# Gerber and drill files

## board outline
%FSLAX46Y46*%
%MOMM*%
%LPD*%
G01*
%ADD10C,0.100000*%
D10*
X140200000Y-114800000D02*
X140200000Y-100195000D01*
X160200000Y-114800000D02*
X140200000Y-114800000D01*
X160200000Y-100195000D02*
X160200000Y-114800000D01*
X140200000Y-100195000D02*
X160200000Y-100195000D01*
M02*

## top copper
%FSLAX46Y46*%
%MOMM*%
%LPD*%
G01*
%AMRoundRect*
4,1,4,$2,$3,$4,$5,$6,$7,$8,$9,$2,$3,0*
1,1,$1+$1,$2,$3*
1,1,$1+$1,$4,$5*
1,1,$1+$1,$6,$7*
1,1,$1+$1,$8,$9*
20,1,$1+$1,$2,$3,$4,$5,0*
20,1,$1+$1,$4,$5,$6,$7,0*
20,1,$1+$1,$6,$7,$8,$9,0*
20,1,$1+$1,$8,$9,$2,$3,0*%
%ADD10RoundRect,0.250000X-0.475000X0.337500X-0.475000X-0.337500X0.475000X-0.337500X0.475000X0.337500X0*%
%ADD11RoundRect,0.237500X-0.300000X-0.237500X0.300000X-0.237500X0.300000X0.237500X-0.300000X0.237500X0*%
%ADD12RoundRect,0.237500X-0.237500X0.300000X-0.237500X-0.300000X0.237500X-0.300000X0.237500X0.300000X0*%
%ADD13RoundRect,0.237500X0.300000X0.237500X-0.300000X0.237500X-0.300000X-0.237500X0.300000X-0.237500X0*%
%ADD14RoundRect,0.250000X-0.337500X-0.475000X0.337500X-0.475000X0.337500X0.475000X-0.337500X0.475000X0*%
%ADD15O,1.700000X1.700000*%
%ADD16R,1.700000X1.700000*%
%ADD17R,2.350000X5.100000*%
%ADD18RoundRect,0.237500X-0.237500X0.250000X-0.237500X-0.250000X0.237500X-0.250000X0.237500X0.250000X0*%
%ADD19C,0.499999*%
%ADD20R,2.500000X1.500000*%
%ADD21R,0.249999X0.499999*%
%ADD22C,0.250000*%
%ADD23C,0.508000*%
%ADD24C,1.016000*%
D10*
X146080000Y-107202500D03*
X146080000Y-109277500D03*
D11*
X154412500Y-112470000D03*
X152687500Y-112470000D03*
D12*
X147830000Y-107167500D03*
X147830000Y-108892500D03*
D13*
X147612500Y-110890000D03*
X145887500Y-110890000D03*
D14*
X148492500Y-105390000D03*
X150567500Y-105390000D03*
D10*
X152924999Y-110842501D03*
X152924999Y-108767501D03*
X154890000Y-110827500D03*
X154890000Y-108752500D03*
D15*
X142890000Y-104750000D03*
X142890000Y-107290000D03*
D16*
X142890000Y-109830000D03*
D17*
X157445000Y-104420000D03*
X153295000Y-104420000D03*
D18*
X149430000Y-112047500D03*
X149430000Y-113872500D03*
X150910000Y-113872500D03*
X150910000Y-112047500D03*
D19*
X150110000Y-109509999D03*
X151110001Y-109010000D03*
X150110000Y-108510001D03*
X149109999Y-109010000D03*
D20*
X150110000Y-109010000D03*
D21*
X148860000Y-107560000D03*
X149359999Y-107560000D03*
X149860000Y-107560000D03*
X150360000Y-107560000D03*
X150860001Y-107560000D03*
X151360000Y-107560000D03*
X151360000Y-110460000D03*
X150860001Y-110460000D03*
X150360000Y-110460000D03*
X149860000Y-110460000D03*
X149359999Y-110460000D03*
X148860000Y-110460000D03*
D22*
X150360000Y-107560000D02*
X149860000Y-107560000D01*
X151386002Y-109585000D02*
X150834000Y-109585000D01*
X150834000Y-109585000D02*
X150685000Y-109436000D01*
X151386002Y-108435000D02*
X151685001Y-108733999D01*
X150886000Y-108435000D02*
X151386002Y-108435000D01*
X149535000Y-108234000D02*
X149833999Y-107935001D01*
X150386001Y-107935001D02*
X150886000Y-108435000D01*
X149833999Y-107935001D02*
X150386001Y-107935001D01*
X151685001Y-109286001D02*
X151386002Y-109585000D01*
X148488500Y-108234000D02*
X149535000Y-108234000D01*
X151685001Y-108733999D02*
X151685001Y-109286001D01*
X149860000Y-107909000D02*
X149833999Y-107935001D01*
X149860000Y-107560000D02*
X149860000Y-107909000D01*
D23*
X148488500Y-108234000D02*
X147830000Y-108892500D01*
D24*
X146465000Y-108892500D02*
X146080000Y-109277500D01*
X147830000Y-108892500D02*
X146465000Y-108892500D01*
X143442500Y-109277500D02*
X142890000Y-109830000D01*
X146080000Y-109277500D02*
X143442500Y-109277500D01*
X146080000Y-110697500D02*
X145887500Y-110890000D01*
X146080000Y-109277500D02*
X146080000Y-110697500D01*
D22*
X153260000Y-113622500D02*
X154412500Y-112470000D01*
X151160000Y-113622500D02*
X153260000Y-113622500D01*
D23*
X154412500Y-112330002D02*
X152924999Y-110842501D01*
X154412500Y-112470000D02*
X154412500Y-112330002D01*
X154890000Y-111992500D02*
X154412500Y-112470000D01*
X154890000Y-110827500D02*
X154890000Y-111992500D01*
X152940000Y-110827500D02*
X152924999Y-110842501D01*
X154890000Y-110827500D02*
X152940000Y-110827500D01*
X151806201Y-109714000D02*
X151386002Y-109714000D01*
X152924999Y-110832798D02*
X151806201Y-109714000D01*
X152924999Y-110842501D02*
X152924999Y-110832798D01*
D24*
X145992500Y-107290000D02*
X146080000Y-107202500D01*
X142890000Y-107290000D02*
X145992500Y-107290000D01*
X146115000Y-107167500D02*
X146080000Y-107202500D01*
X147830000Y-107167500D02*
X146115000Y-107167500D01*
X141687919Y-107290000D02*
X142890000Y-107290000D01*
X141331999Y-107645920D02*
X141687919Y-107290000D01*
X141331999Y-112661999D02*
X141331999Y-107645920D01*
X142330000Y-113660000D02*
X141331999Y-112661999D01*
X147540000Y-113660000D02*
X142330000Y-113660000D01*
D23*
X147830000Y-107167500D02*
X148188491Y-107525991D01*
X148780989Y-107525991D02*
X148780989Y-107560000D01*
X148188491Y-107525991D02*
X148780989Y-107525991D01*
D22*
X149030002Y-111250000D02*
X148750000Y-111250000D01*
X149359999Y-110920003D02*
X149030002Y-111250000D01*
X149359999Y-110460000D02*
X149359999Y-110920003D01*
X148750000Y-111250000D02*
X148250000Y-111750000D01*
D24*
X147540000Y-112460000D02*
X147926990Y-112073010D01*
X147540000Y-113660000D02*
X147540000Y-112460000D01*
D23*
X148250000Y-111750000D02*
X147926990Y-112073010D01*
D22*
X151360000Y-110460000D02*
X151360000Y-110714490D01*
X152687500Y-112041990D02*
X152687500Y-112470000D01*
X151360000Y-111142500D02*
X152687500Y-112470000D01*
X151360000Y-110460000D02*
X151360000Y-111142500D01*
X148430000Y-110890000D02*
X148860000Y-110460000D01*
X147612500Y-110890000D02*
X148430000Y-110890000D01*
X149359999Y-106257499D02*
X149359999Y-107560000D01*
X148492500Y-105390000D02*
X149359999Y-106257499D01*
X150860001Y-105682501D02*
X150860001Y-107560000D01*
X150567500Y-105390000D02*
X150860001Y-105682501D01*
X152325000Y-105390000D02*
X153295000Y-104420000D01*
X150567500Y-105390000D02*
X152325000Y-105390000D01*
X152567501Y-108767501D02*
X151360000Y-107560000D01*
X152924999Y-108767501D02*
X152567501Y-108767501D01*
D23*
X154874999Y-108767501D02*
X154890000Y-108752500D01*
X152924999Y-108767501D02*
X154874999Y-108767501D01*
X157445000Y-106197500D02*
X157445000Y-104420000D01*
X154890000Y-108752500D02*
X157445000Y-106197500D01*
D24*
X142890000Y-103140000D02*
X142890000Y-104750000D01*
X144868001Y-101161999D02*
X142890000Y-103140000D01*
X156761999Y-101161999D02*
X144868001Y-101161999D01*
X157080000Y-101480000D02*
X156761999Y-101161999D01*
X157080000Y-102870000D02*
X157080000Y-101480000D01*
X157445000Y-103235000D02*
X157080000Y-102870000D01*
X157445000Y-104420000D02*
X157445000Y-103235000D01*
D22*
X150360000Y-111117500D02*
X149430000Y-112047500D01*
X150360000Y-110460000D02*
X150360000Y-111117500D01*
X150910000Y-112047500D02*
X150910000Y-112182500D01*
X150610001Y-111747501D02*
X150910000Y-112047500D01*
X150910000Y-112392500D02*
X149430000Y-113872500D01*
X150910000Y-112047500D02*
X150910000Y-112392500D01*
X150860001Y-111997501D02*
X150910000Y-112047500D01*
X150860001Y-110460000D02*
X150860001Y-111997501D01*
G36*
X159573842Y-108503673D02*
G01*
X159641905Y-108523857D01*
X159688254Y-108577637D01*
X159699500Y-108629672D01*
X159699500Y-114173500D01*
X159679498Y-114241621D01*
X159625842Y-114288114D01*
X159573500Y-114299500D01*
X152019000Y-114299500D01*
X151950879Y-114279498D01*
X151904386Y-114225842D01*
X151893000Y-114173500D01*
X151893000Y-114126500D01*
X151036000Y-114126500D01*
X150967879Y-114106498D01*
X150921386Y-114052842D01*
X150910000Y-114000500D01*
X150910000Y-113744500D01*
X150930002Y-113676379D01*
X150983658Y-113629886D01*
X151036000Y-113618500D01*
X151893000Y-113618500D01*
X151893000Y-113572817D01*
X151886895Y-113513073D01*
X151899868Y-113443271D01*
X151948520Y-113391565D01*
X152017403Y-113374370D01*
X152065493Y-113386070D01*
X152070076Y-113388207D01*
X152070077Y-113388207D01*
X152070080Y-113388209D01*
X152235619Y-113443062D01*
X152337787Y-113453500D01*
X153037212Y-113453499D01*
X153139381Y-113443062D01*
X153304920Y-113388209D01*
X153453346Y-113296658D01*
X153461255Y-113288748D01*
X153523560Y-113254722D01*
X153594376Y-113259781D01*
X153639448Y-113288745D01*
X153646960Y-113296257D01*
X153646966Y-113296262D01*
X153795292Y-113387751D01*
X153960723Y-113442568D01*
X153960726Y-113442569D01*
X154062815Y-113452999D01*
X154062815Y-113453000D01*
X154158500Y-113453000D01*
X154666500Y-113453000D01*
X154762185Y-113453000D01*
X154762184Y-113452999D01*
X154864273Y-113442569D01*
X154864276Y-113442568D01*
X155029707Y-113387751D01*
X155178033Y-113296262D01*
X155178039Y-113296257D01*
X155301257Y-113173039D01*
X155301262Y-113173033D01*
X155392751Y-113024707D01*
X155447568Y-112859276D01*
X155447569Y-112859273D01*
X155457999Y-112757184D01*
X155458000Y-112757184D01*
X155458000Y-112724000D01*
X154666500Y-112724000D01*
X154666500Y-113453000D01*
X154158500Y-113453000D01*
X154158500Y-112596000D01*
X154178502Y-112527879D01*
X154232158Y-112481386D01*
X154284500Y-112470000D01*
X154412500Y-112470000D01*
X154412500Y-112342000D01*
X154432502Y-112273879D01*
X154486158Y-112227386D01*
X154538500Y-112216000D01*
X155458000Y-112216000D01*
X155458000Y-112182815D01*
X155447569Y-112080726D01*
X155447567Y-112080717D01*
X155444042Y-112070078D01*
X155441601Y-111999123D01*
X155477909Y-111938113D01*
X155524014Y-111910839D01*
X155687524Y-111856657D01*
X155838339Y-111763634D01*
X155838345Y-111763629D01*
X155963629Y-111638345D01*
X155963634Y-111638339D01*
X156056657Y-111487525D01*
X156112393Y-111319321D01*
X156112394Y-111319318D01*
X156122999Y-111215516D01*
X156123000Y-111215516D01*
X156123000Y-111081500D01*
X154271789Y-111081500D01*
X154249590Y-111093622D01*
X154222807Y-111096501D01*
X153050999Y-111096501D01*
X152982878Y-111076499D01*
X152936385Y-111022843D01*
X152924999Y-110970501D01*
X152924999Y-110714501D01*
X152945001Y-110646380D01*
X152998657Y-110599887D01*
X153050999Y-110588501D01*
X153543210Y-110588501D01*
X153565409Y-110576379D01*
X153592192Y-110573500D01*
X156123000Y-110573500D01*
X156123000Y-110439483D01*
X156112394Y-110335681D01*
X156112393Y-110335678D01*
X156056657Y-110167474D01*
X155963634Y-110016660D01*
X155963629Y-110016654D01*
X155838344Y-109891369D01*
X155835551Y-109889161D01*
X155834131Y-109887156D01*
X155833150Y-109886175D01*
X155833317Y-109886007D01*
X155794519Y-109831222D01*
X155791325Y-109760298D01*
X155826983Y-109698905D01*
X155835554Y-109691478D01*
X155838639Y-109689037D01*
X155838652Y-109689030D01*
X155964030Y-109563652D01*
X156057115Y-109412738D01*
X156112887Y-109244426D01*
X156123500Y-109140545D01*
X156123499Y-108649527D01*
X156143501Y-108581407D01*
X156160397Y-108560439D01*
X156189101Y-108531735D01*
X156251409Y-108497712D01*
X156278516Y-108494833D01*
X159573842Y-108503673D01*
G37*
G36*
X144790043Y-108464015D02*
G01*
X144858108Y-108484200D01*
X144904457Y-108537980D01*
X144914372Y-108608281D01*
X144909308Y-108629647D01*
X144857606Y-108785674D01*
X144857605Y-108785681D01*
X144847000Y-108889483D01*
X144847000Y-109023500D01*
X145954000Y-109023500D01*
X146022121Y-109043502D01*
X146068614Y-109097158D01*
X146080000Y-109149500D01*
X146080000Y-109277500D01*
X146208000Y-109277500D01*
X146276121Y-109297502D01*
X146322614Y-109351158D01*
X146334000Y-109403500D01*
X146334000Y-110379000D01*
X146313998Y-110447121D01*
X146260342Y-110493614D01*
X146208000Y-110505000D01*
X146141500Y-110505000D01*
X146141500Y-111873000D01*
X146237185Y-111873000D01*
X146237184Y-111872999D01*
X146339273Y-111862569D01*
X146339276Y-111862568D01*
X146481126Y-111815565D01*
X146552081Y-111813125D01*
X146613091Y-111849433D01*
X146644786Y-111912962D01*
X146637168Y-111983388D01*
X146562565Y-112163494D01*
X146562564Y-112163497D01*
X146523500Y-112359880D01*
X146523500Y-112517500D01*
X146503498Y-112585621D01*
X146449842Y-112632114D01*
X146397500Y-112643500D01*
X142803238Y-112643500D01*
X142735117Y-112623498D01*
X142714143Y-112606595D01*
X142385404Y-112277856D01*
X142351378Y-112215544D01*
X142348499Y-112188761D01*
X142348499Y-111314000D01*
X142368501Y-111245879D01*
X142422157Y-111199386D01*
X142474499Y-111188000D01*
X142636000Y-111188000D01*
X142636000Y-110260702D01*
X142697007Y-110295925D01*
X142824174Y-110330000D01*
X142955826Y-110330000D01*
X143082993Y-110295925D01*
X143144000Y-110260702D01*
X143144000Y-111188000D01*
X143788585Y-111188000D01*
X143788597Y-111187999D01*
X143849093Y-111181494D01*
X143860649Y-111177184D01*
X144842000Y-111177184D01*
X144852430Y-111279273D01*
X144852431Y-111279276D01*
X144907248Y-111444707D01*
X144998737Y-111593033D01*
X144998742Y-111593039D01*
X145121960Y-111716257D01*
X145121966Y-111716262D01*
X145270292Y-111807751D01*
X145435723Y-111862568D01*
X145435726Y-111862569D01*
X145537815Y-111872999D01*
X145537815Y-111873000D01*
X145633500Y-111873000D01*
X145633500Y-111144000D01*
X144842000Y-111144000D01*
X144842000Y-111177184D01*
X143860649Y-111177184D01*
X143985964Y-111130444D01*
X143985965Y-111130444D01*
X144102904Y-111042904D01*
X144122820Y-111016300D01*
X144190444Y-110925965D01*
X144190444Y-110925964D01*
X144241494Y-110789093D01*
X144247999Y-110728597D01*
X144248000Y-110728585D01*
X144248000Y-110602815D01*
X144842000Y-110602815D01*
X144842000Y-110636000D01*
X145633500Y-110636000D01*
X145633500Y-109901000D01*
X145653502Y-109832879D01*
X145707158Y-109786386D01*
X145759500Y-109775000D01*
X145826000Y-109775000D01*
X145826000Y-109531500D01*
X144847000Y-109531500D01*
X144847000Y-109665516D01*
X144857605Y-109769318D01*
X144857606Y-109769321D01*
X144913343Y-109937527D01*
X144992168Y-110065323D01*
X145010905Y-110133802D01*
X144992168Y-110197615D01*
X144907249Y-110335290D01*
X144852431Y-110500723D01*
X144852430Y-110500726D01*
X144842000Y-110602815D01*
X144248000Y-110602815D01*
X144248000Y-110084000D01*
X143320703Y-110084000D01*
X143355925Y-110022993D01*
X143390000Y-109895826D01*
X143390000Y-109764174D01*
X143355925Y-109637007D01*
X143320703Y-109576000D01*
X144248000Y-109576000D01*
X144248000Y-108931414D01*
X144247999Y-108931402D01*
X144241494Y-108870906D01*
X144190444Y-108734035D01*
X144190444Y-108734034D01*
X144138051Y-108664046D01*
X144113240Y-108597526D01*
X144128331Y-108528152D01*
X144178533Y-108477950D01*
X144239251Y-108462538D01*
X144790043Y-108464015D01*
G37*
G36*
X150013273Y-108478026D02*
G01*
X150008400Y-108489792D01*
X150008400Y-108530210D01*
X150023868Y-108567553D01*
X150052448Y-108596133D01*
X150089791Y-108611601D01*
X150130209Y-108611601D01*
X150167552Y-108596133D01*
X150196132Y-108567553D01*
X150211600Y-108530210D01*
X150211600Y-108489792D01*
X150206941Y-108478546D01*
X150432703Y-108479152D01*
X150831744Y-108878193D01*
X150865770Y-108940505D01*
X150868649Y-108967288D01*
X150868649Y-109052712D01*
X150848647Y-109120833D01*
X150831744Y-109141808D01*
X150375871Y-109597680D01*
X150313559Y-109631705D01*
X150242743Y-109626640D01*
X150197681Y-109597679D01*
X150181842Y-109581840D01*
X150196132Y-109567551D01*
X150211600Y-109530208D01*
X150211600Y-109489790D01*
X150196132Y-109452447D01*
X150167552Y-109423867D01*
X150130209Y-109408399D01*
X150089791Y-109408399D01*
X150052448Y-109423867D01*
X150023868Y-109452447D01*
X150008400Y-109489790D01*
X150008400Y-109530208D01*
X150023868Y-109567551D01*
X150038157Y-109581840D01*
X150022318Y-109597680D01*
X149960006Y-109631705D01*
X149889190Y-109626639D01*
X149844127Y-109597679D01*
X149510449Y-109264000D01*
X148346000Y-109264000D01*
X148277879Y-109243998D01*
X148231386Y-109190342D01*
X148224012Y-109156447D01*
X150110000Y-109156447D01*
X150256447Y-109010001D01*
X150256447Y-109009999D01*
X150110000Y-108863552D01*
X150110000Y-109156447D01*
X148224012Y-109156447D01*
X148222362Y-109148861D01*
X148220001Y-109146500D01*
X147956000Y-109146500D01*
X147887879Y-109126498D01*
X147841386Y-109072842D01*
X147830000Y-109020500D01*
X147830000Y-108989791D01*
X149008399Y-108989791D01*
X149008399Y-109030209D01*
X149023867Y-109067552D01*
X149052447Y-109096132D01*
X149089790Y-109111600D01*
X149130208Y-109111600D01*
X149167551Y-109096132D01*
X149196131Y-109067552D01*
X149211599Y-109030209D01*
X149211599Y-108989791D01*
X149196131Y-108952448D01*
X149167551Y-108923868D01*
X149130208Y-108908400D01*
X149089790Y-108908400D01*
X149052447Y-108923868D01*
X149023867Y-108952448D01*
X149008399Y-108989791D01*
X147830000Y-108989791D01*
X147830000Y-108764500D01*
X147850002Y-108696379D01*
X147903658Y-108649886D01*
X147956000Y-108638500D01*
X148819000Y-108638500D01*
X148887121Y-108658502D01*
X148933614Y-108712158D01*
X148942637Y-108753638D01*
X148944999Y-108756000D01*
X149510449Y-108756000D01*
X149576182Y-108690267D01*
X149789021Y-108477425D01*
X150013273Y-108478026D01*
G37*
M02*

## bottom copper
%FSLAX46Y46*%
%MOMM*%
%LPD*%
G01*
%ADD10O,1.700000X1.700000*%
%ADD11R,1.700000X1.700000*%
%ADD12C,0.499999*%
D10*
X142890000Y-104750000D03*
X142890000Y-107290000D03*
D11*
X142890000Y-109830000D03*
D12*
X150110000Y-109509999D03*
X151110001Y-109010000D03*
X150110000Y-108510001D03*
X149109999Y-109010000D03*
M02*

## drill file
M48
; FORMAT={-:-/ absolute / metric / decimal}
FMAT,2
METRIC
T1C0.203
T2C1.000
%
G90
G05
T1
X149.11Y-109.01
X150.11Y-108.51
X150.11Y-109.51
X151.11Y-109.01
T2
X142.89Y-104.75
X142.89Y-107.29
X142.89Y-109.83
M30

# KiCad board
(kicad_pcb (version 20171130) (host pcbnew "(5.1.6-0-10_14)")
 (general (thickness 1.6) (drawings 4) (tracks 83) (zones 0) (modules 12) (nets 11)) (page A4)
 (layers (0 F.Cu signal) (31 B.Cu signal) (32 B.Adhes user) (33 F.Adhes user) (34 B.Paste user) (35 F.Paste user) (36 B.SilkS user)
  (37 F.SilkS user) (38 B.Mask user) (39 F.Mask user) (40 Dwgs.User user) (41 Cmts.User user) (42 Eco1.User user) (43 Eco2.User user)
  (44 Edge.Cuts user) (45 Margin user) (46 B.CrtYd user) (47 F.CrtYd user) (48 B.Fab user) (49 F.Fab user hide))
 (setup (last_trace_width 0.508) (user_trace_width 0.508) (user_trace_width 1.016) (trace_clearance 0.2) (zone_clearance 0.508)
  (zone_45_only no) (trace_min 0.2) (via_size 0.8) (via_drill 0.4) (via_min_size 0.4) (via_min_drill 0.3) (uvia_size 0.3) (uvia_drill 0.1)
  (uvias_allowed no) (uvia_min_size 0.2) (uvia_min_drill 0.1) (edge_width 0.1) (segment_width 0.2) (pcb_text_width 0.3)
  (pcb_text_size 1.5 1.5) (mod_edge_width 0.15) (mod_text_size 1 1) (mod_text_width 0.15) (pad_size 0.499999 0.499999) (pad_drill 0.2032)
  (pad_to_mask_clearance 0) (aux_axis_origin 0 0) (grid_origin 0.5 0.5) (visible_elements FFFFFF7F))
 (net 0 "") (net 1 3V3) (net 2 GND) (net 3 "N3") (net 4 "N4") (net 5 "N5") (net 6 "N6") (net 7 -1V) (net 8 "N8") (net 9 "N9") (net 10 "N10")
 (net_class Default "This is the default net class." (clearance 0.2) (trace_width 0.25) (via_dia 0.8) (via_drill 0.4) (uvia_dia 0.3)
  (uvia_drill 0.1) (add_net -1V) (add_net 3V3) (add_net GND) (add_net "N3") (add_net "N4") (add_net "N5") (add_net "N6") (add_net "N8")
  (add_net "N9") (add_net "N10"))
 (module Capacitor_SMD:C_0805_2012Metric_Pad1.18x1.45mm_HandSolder (layer F.Cu) (at 146.08 108.24 270)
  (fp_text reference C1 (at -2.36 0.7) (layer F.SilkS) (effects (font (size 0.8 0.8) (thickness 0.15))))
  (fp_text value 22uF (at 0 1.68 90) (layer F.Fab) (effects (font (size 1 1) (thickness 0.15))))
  (pad 1 smd roundrect (at -1.0375 0 270) (size 1.175 1.45) (layers F.Cu F.Paste F.Mask) (roundrect_rratio 0.212766) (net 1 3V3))
  (pad 2 smd roundrect (at 1.0375 0 270) (size 1.175 1.45) (layers F.Cu F.Paste F.Mask) (roundrect_rratio 0.212766) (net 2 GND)))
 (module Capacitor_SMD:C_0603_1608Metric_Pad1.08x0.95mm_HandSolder (layer F.Cu) (at 153.55 112.47)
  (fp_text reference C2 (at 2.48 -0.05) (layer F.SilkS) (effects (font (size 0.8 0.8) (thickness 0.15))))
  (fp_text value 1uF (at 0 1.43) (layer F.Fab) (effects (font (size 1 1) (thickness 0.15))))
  (pad 2 smd roundrect (at 0.8625 0) (size 1.075 0.95) (layers F.Cu F.Paste F.Mask) (roundrect_rratio 0.25) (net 2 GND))
  (pad 1 smd roundrect (at -0.8625 0) (size 1.075 0.95) (layers F.Cu F.Paste F.Mask) (roundrect_rratio 0.25) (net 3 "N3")))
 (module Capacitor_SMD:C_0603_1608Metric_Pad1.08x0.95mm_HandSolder (layer F.Cu) (at 147.83 108.03 270)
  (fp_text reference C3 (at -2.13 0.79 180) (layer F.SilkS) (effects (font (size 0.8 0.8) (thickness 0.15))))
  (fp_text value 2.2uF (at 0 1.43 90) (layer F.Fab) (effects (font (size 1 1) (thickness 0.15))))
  (pad 1 smd roundrect (at -0.8625 0 270) (size 1.075 0.95) (layers F.Cu F.Paste F.Mask) (roundrect_rratio 0.25) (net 1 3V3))
  (pad 2 smd roundrect (at 0.8625 0 270) (size 1.075 0.95) (layers F.Cu F.Paste F.Mask) (roundrect_rratio 0.25) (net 2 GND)))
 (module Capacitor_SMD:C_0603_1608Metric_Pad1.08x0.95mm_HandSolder (layer F.Cu) (at 146.75 110.89 180)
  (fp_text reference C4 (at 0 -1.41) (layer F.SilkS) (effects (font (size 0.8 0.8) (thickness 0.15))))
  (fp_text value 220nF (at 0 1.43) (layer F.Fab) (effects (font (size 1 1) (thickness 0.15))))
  (pad 1 smd roundrect (at -0.8625 0 180) (size 1.075 0.95) (layers F.Cu F.Paste F.Mask) (roundrect_rratio 0.25) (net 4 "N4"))
  (pad 2 smd roundrect (at 0.8625 0 180) (size 1.075 0.95) (layers F.Cu F.Paste F.Mask) (roundrect_rratio 0.25) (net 2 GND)))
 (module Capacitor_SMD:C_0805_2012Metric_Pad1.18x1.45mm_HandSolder (layer F.Cu) (at 149.53 105.39)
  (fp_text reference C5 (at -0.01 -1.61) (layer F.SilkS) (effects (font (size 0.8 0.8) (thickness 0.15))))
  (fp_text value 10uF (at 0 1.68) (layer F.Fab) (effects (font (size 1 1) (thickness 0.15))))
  (pad 1 smd roundrect (at -1.0375 0) (size 1.175 1.45) (layers F.Cu F.Paste F.Mask) (roundrect_rratio 0.212766) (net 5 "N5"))
  (pad 2 smd roundrect (at 1.0375 0) (size 1.175 1.45) (layers F.Cu F.Paste F.Mask) (roundrect_rratio 0.212766) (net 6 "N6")))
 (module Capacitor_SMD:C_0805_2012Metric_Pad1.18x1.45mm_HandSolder (layer F.Cu) (at 152.924999 109.805001 270)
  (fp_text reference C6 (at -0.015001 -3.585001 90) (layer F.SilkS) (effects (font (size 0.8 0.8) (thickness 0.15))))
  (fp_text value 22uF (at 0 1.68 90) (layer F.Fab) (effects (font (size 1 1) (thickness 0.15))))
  (pad 2 smd roundrect (at 1.0375 0 270) (size 1.175 1.45) (layers F.Cu F.Paste F.Mask) (roundrect_rratio 0.212766) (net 2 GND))
  (pad 1 smd roundrect (at -1.0375 0 270) (size 1.175 1.45) (layers F.Cu F.Paste F.Mask) (roundrect_rratio 0.212766) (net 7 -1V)))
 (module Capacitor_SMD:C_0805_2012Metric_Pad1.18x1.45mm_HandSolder (layer F.Cu) (at 154.89 109.79 270)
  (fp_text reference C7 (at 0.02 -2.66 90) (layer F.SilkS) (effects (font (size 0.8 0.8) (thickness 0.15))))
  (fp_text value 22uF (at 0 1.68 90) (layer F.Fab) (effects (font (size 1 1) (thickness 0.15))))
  (pad 2 smd roundrect (at 1.0375 0 270) (size 1.175 1.45) (layers F.Cu F.Paste F.Mask) (roundrect_rratio 0.212766) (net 2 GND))
  (pad 1 smd roundrect (at -1.0375 0 270) (size 1.175 1.45) (layers F.Cu F.Paste F.Mask) (roundrect_rratio 0.212766) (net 7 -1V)))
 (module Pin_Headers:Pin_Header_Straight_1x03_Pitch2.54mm (layer F.Cu) (at 142.89 109.83 180)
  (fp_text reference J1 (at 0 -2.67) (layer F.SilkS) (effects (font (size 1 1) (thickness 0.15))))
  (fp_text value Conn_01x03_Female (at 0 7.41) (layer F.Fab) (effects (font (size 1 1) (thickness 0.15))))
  (pad 3 thru_hole oval (at 0 5.08 180) (size 1.7 1.7) (drill 1) (layers *.Cu *.Mask) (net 7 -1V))
  (pad 2 thru_hole oval (at 0 2.54 180) (size 1.7 1.7) (drill 1) (layers *.Cu *.Mask) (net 1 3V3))
  (pad 1 thru_hole rect (at 0 0 180) (size 1.7 1.7) (drill 1) (layers *.Cu *.Mask) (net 2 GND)))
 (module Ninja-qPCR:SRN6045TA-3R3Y (layer F.Cu) (at 155.37 104.42)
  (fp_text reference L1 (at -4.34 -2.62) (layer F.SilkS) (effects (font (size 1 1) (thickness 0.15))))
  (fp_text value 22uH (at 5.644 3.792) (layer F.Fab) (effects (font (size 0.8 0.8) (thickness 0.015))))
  (pad 2 smd rect (at 2.075 0) (size 2.35 5.1) (layers F.Cu F.Paste F.Mask) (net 7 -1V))
  (pad 1 smd rect (at -2.075 0) (size 2.35 5.1) (layers F.Cu F.Paste F.Mask) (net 6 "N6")))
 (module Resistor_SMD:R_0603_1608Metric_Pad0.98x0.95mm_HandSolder (layer F.Cu) (at 149.43 112.96 270)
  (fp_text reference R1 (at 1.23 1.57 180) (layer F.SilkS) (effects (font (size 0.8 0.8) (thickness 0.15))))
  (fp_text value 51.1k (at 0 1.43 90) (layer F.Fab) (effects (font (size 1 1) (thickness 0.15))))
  (pad 1 smd roundrect (at -0.9125 0 270) (size 0.975 0.95) (layers F.Cu F.Paste F.Mask) (roundrect_rratio 0.25) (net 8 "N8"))
  (pad 2 smd roundrect (at 0.9125 0 270) (size 0.975 0.95) (layers F.Cu F.Paste F.Mask) (roundrect_rratio 0.25) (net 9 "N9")))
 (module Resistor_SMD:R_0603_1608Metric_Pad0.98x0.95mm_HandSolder (layer F.Cu) (at 150.91 112.96 270)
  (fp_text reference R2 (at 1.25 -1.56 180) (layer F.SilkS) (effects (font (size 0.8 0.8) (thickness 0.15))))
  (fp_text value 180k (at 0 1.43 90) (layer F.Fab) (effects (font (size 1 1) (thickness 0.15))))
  (pad 2 smd roundrect (at 0.9125 0 270) (size 0.975 0.95) (layers F.Cu F.Paste F.Mask) (roundrect_rratio 0.25) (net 2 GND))
  (pad 1 smd roundrect (at -0.9125 0 270) (size 0.975 0.95) (layers F.Cu F.Paste F.Mask) (roundrect_rratio 0.25) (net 9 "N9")))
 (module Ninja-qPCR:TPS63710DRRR (layer F.Cu) (at 150.11 109.01 90)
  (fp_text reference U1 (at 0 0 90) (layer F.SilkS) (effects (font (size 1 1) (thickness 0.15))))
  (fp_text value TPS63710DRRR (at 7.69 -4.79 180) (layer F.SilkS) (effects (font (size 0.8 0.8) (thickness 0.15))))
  (pad V thru_hole circle (at -0.499999 0 90) (size 0.499999 0.499999) (drill 0.2032) (layers *.Cu *.Mask) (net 2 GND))
  (pad V thru_hole circle (at 0 1.000001 90) (size 0.499999 0.499999) (drill 0.2032) (layers *.Cu *.Mask) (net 2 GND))
  (pad V thru_hole circle (at 0.499999 0 90) (size 0.499999 0.499999) (drill 0.2032) (layers *.Cu *.Mask) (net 2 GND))
  (pad V thru_hole circle (at 0 -1.000001 90) (size 0.499999 0.499999) (drill 0.2032) (layers *.Cu *.Mask) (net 2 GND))
  (pad 13 smd rect (at 0 0 90) (size 1.5 2.5) (layers F.Cu F.Paste F.Mask) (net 2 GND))
  (pad 12 smd rect (at 1.45 -1.25 90) (size 0.499999 0.249999) (layers F.Cu F.Paste F.Mask) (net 1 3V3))
  (pad 11 smd rect (at 1.45 -0.750001 90) (size 0.499999 0.249999) (layers F.Cu F.Paste F.Mask) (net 5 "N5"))
  (pad 10 smd rect (at 1.45 -0.25 90) (size 0.499999 0.249999) (layers F.Cu F.Paste F.Mask) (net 2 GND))
  (pad 9 smd rect (at 1.45 0.25 90) (size 0.499999 0.249999) (layers F.Cu F.Paste F.Mask) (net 2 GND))
  (pad 8 smd rect (at 1.45 0.750001 90) (size 0.499999 0.249999) (layers F.Cu F.Paste F.Mask) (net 6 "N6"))
  (pad 7 smd rect (at 1.45 1.25 90) (size 0.499999 0.249999) (layers F.Cu F.Paste F.Mask) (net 7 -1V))
  (pad 6 smd rect (at -1.45 1.25 90) (size 0.499999 0.249999) (layers F.Cu F.Paste F.Mask) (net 3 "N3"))
  (pad 5 smd rect (at -1.45 0.750001 90) (size 0.499999 0.249999) (layers F.Cu F.Paste F.Mask) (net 9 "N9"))
  (pad 4 smd rect (at -1.45 0.25 90) (size 0.499999 0.249999) (layers F.Cu F.Paste F.Mask) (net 8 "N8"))
  (pad 3 smd rect (at -1.45 -0.25 90) (size 0.499999 0.249999) (layers F.Cu F.Paste F.Mask) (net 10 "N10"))
  (pad 2 smd rect (at -1.45 -0.750001 90) (size 0.499999 0.249999) (layers F.Cu F.Paste F.Mask) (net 1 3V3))
  (pad 1 smd rect (at -1.45 -1.25 90) (size 0.499999 0.249999) (layers F.Cu F.Paste F.Mask) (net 4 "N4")))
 (gr_line (start 140.2 114.8) (end 140.2 100.195) (layer Edge.Cuts) (width 0.1))
 (gr_line (start 160.2 114.8) (end 140.2 114.8) (layer Edge.Cuts) (width 0.1))
 (gr_line (start 160.2 100.195) (end 160.2 114.8) (layer Edge.Cuts) (width 0.1))
 (gr_line (start 140.2 100.195) (end 160.2 100.195) (layer Edge.Cuts) (width 0.1))
 (segment (start 150.36 107.56) (end 149.86 107.56) (width 0.25) (layer F.Cu) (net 2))
 (segment (start 151.386002 109.585) (end 150.834 109.585) (width 0.25) (layer F.Cu) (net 2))
 (segment (start 150.834 109.585) (end 150.685 109.436) (width 0.25) (layer F.Cu) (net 2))
 (segment (start 151.386002 108.435) (end 151.685001 108.733999) (width 0.25) (layer F.Cu) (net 2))
 (segment (start 150.886 108.435) (end 151.386002 108.435) (width 0.25) (layer F.Cu) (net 2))
 (segment (start 149.535 108.234) (end 149.833999 107.935001) (width 0.25) (layer F.Cu) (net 2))
 (segment (start 150.386001 107.935001) (end 150.886 108.435) (width 0.25) (layer F.Cu) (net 2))
 (segment (start 149.833999 107.935001) (end 150.386001 107.935001) (width 0.25) (layer F.Cu) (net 2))
 (segment (start 151.685001 109.286001) (end 151.386002 109.585) (width 0.25) (layer F.Cu) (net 2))
 (segment (start 148.4885 108.234) (end 149.535 108.234) (width 0.25) (layer F.Cu) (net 2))
 (segment (start 151.685001 108.733999) (end 151.685001 109.286001) (width 0.25) (layer F.Cu) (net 2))
 (segment (start 149.86 107.909) (end 149.833999 107.935001) (width 0.25) (layer F.Cu) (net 2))
 (segment (start 149.86 107.56) (end 149.86 107.909) (width 0.25) (layer F.Cu) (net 2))
 (segment (start 148.4885 108.234) (end 147.83 108.8925) (width 0.508) (layer F.Cu) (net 2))
 (segment (start 146.465 108.8925) (end 146.08 109.2775) (width 1.016) (layer F.Cu) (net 2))
 (segment (start 147.83 108.8925) (end 146.465 108.8925) (width 1.016) (layer F.Cu) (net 2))
 (segment (start 143.4425 109.2775) (end 142.89 109.83) (width 1.016) (layer F.Cu) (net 2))
 (segment (start 146.08 109.2775) (end 143.4425 109.2775) (width 1.016) (layer F.Cu) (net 2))
 (segment (start 146.08 110.6975) (end 145.8875 110.89) (width 1.016) (layer F.Cu) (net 2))
 (segment (start 146.08 109.2775) (end 146.08 110.6975) (width 1.016) (layer F.Cu) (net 2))
 (segment (start 153.26 113.6225) (end 154.4125 112.47) (width 0.25) (layer F.Cu) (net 2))
 (segment (start 151.16 113.6225) (end 153.26 113.6225) (width 0.25) (layer F.Cu) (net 2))
 (segment (start 154.4125 112.330002) (end 152.924999 110.842501) (width 0.508) (layer F.Cu) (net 2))
 (segment (start 154.4125 112.47) (end 154.4125 112.330002) (width 0.508) (layer F.Cu) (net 2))
 (segment (start 154.89 111.9925) (end 154.4125 112.47) (width 0.508) (layer F.Cu) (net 2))
 (segment (start 154.89 110.8275) (end 154.89 111.9925) (width 0.508) (layer F.Cu) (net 2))
 (segment (start 152.94 110.8275) (end 152.924999 110.842501) (width 0.508) (layer F.Cu) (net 2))
 (segment (start 154.89 110.8275) (end 152.94 110.8275) (width 0.508) (layer F.Cu) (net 2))
 (segment (start 151.806201 109.714) (end 151.386002 109.714) (width 0.508) (layer F.Cu) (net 2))
 (segment (start 152.924999 110.832798) (end 151.806201 109.714) (width 0.508) (layer F.Cu) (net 2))
 (segment (start 152.924999 110.842501) (end 152.924999 110.832798) (width 0.508) (layer F.Cu) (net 2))
 (segment (start 145.9925 107.29) (end 146.08 107.2025) (width 1.016) (layer F.Cu) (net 1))
 (segment (start 142.89 107.29) (end 145.9925 107.29) (width 1.016) (layer F.Cu) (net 1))
 (segment (start 146.115 107.1675) (end 146.08 107.2025) (width 1.016) (layer F.Cu) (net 1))
 (segment (start 147.83 107.1675) (end 146.115 107.1675) (width 1.016) (layer F.Cu) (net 1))
 (segment (start 141.687919 107.29) (end 142.89 107.29) (width 1.016) (layer F.Cu) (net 1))
 (segment (start 141.331999 107.64592) (end 141.687919 107.29) (width 1.016) (layer F.Cu) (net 1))
 (segment (start 141.331999 112.661999) (end 141.331999 107.64592) (width 1.016) (layer F.Cu) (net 1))
 (segment (start 142.33 113.66) (end 141.331999 112.661999) (width 1.016) (layer F.Cu) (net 1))
 (segment (start 147.54 113.66) (end 142.33 113.66) (width 1.016) (layer F.Cu) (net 1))
 (segment (start 147.83 107.1675) (end 148.188491 107.525991) (width 0.508) (layer F.Cu) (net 1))
 (segment (start 148.780989 107.525991) (end 148.780989 107.56) (width 0.508) (layer F.Cu) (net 1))
 (segment (start 148.188491 107.525991) (end 148.780989 107.525991) (width 0.508) (layer F.Cu) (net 1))
 (segment (start 149.030002 111.25) (end 148.75 111.25) (width 0.25) (layer F.Cu) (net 1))
 (segment (start 149.359999 110.920003) (end 149.030002 111.25) (width 0.25) (layer F.Cu) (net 1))
 (segment (start 149.359999 110.46) (end 149.359999 110.920003) (width 0.25) (layer F.Cu) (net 1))
 (segment (start 148.75 111.25) (end 148.25 111.75) (width 0.25) (layer F.Cu) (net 1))
 (segment (start 147.54 112.46) (end 147.92699 112.07301) (width 1.016) (layer F.Cu) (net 1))
 (segment (start 147.54 113.66) (end 147.54 112.46) (width 1.016) (layer F.Cu) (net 1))
 (segment (start 148.25 111.75) (end 147.92699 112.07301) (width 0.508) (layer F.Cu) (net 1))
 (segment (start 151.36 110.46) (end 151.36 110.71449) (width 0.25) (layer F.Cu) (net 3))
 (segment (start 152.6875 112.04199) (end 152.6875 112.47) (width 0.25) (layer F.Cu) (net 3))
 (segment (start 151.36 111.1425) (end 152.6875 112.47) (width 0.25) (layer F.Cu) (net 3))
 (segment (start 151.36 110.46) (end 151.36 111.1425) (width 0.25) (layer F.Cu) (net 3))
 (segment (start 148.43 110.89) (end 148.86 110.46) (width 0.25) (layer F.Cu) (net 4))
 (segment (start 147.6125 110.89) (end 148.43 110.89) (width 0.25) (layer F.Cu) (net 4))
 (segment (start 149.359999 106.257499) (end 149.359999 107.56) (width 0.25) (layer F.Cu) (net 5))
 (segment (start 148.4925 105.39) (end 149.359999 106.257499) (width 0.25) (layer F.Cu) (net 5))
 (segment (start 150.860001 105.682501) (end 150.860001 107.56) (width 0.25) (layer F.Cu) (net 6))
 (segment (start 150.5675 105.39) (end 150.860001 105.682501) (width 0.25) (layer F.Cu) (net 6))
 (segment (start 152.325 105.39) (end 153.295 104.42) (width 0.25) (layer F.Cu) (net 6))
 (segment (start 150.5675 105.39) (end 152.325 105.39) (width 0.25) (layer F.Cu) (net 6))
 (segment (start 152.567501 108.767501) (end 151.36 107.56) (width 0.25) (layer F.Cu) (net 7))
 (segment (start 152.924999 108.767501) (end 152.567501 108.767501) (width 0.25) (layer F.Cu) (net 7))
 (segment (start 154.874999 108.767501) (end 154.89 108.7525) (width 0.508) (layer F.Cu) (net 7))
 (segment (start 152.924999 108.767501) (end 154.874999 108.767501) (width 0.508) (layer F.Cu) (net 7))
 (segment (start 157.445 106.1975) (end 157.445 104.42) (width 0.508) (layer F.Cu) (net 7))
 (segment (start 154.89 108.7525) (end 157.445 106.1975) (width 0.508) (layer F.Cu) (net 7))
 (segment (start 142.89 103.14) (end 142.89 104.75) (width 1.016) (layer F.Cu) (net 7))
 (segment (start 144.868001 101.161999) (end 142.89 103.14) (width 1.016) (layer F.Cu) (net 7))
 (segment (start 156.761999 101.161999) (end 144.868001 101.161999) (width 1.016) (layer F.Cu) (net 7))
 (segment (start 157.08 101.48) (end 156.761999 101.161999) (width 1.016) (layer F.Cu) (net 7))
 (segment (start 157.08 102.87) (end 157.08 101.48) (width 1.016) (layer F.Cu) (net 7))
 (segment (start 157.445 103.235) (end 157.08 102.87) (width 1.016) (layer F.Cu) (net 7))
 (segment (start 157.445 104.42) (end 157.445 103.235) (width 1.016) (layer F.Cu) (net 7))
 (segment (start 150.36 111.1175) (end 149.43 112.0475) (width 0.25) (layer F.Cu) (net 8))
 (segment (start 150.36 110.46) (end 150.36 111.1175) (width 0.25) (layer F.Cu) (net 8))
 (segment (start 150.91 112.0475) (end 150.91 112.1825) (width 0.25) (layer F.Cu) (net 9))
 (segment (start 150.610001 111.747501) (end 150.91 112.0475) (width 0.25) (layer F.Cu) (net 9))
 (segment (start 150.91 112.3925) (end 149.43 113.8725) (width 0.25) (layer F.Cu) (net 9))
 (segment (start 150.91 112.0475) (end 150.91 112.3925) (width 0.25) (layer F.Cu) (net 9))
 (segment (start 150.860001 111.997501) (end 150.91 112.0475) (width 0.25) (layer F.Cu) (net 9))
 (segment (start 150.860001 110.46) (end 150.860001 111.997501) (width 0.25) (layer F.Cu) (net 9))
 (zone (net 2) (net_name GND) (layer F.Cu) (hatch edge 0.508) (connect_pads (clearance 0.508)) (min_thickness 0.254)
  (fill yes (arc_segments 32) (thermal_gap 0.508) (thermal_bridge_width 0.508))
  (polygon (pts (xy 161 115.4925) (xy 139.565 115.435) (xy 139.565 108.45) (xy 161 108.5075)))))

